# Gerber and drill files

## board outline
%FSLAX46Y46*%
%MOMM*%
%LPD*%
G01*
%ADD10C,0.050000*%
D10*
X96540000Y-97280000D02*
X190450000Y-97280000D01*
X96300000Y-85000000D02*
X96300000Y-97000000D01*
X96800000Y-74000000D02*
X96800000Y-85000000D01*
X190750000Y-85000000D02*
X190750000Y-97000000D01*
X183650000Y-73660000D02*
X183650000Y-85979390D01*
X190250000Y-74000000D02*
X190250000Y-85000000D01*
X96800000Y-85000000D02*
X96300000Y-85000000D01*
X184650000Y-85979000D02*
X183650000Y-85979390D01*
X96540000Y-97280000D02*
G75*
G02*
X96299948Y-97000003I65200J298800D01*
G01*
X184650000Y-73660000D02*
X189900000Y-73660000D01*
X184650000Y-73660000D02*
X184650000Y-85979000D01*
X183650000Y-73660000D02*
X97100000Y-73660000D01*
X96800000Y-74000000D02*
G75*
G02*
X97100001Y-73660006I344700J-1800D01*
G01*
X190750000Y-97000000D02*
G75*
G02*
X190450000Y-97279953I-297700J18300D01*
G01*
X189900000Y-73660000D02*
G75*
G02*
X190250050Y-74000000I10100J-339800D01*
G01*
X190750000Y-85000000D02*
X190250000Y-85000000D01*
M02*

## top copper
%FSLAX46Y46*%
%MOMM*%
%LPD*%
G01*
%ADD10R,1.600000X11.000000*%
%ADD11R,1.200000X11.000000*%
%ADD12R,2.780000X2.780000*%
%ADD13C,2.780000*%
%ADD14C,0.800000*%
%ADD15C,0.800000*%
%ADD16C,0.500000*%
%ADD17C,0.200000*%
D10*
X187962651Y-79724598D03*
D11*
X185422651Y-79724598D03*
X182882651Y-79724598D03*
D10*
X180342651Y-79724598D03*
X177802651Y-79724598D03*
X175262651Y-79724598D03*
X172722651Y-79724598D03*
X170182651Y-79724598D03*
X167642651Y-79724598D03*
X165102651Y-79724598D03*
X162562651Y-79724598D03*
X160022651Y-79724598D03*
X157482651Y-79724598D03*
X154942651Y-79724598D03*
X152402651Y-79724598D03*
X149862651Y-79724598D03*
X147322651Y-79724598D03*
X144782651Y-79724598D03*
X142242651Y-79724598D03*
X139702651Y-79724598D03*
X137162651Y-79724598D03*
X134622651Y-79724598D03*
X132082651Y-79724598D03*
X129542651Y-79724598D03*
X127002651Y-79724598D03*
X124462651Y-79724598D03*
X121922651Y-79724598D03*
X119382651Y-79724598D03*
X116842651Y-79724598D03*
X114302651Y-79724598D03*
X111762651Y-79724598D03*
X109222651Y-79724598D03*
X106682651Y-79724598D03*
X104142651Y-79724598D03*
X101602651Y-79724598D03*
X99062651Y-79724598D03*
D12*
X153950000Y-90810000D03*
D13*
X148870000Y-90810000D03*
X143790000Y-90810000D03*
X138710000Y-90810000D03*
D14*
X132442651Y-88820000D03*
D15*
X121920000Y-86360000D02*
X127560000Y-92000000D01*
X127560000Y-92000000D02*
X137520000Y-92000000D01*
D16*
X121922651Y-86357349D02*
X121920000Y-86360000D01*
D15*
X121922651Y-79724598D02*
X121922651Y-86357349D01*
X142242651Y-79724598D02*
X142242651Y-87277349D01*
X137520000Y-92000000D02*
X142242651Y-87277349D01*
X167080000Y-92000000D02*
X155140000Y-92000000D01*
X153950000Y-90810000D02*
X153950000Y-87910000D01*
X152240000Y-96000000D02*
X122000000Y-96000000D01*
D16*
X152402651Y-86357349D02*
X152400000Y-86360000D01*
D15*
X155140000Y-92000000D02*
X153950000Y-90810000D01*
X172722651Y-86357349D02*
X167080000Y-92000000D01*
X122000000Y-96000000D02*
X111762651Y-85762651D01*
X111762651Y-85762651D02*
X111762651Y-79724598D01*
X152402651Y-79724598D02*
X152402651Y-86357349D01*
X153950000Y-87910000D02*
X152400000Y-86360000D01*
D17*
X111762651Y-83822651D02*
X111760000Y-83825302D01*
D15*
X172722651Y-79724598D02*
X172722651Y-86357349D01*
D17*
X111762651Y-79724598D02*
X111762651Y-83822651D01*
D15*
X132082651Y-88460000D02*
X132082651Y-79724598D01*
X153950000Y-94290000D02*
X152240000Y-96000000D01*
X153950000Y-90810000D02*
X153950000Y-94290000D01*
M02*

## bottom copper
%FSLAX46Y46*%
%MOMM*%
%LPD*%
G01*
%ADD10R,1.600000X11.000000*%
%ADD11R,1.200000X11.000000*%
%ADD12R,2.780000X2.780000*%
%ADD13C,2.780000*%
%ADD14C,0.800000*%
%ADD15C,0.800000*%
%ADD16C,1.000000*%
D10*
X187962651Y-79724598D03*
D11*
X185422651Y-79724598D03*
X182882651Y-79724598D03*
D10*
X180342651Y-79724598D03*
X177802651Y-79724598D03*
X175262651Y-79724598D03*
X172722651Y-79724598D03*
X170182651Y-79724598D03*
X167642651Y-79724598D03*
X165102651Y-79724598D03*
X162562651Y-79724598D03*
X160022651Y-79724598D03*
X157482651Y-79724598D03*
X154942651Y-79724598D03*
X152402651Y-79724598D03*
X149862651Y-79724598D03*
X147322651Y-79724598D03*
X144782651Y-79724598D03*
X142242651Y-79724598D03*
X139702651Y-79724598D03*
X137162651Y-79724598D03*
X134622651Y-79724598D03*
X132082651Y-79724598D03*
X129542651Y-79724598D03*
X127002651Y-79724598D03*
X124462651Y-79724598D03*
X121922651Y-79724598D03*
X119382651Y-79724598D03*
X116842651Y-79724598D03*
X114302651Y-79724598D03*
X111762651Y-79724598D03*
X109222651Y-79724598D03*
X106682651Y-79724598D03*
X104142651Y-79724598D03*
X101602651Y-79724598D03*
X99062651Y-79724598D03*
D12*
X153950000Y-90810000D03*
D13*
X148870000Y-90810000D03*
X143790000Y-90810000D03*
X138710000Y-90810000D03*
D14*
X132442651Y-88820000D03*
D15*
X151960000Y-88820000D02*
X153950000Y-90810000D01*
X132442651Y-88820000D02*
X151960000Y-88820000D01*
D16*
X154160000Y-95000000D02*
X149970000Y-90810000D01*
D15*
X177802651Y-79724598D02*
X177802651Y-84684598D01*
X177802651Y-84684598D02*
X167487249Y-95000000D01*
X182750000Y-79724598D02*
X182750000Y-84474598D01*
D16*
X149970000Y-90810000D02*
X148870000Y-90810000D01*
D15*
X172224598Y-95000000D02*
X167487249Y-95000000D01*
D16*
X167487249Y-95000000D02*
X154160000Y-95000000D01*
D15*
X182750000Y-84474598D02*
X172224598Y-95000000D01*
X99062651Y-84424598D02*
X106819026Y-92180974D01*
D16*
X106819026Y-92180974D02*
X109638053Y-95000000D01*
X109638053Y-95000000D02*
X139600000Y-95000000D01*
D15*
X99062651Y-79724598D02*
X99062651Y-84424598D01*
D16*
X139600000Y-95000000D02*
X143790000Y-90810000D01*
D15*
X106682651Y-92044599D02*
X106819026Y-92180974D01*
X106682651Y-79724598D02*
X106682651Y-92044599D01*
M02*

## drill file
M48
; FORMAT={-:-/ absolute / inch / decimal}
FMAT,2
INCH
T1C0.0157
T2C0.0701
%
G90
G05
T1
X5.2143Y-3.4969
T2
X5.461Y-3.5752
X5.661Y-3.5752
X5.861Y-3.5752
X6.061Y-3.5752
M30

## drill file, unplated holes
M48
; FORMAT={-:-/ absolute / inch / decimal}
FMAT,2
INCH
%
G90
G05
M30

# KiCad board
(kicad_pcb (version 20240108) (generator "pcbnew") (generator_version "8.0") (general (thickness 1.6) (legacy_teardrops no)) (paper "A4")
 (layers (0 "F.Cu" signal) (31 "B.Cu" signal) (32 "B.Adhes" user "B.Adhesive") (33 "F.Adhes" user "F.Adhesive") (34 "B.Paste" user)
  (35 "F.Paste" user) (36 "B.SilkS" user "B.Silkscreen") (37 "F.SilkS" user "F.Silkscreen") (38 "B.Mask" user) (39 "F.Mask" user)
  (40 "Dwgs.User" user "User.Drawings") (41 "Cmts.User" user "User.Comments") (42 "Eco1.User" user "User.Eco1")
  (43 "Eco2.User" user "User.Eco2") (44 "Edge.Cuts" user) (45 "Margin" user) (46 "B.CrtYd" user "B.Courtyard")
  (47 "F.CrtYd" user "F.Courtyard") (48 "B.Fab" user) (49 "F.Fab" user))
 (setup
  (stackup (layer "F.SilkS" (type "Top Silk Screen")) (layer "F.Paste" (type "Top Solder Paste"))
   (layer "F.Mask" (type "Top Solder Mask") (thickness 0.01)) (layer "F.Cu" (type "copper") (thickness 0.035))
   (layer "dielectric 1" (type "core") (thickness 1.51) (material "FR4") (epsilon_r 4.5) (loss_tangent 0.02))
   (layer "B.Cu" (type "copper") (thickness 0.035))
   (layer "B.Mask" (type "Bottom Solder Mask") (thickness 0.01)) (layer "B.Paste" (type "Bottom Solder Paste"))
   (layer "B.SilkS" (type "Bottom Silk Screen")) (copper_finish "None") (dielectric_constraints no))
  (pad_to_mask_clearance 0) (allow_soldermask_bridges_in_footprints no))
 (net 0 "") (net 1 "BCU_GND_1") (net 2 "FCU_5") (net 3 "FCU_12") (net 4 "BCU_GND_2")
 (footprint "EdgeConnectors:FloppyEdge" (layer "F.Cu") (at 167.642651 87.344598)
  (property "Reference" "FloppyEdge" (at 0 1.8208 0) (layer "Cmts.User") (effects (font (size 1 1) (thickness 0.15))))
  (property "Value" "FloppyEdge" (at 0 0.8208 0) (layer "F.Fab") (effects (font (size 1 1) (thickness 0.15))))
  (pad "1" smd rect (at 20.32 -7.62) (size 1.6 11) (layers "F.Cu" "F.Paste" "F.Mask"))
  (pad "2" smd rect (at 20.32 -7.62) (size 1.6 11) (layers "B.Cu" "B.Paste" "B.Mask"))
  (pad "3" smd rect (at 17.78 -7.62) (size 1.2 11) (layers "F.Cu" "F.Paste" "F.Mask"))
  (pad "4" smd rect (at 17.78 -7.62) (size 1.2 11) (layers "B.Cu" "B.Paste" "B.Mask"))
  (pad "5" smd rect (at 15.24 -7.62) (size 1.2 11) (layers "F.Cu" "F.Paste" "F.Mask"))
  (pad "6" smd rect (at 15.24 -7.62) (size 1.2 11) (layers "B.Cu" "B.Paste" "B.Mask") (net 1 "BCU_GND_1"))
  (pad "7" smd rect (at 12.7 -7.62) (size 1.6 11) (layers "F.Cu" "F.Paste" "F.Mask"))
  (pad "8" smd rect (at 12.7 -7.62) (size 1.6 11) (layers "B.Cu" "B.Paste" "B.Mask"))
  (pad "9" smd rect (at 10.16 -7.62) (size 1.6 11) (layers "F.Cu" "F.Paste" "F.Mask"))
  (pad "10" smd rect (at 10.16 -7.62) (size 1.6 11) (layers "B.Cu" "B.Paste" "B.Mask") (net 1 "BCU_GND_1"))
  (pad "11" smd rect (at 7.62 -7.62) (size 1.6 11) (layers "F.Cu" "F.Paste" "F.Mask"))
  (pad "12" smd rect (at 7.62 -7.62) (size 1.6 11) (layers "B.Cu" "B.Paste" "B.Mask"))
  (pad "13" smd rect (at 5.08 -7.62) (size 1.6 11) (layers "F.Cu" "F.Paste" "F.Mask") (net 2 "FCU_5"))
  (pad "14" smd rect (at 5.08 -7.62) (size 1.6 11) (layers "B.Cu" "B.Paste" "B.Mask"))
  (pad "15" smd rect (at 2.54 -7.62) (size 1.6 11) (layers "F.Cu" "F.Paste" "F.Mask"))
  (pad "16" smd rect (at 2.54 -7.62) (size 1.6 11) (layers "B.Cu" "B.Paste" "B.Mask"))
  (pad "17" smd rect (at 0 -7.62) (size 1.6 11) (layers "F.Cu" "F.Paste" "F.Mask"))
  (pad "18" smd rect (at 0 -7.62) (size 1.6 11) (layers "B.Cu" "B.Paste" "B.Mask"))
  (pad "19" smd rect (at -2.54 -7.62) (size 1.6 11) (layers "F.Cu" "F.Paste" "F.Mask"))
  (pad "20" smd rect (at -2.54 -7.62) (size 1.6 11) (layers "B.Cu" "B.Paste" "B.Mask"))
  (pad "21" smd rect (at -5.08 -7.62) (size 1.6 11) (layers "F.Cu" "F.Paste" "F.Mask"))
  (pad "22" smd rect (at -5.08 -7.62) (size 1.6 11) (layers "B.Cu" "B.Paste" "B.Mask"))
  (pad "23" smd rect (at -7.62 -7.62) (size 1.6 11) (layers "F.Cu" "F.Paste" "F.Mask"))
  (pad "24" smd rect (at -7.62 -7.62) (size 1.6 11) (layers "B.Cu" "B.Paste" "B.Mask"))
  (pad "25" smd rect (at -10.16 -7.62) (size 1.6 11) (layers "F.Cu" "F.Paste" "F.Mask"))
  (pad "26" smd rect (at -10.16 -7.62) (size 1.6 11) (layers "B.Cu" "B.Paste" "B.Mask"))
  (pad "27" smd rect (at -12.7 -7.62) (size 1.6 11) (layers "F.Cu" "F.Paste" "F.Mask"))
  (pad "28" smd rect (at -12.7 -7.62) (size 1.6 11) (layers "B.Cu" "B.Paste" "B.Mask"))
  (pad "29" smd rect (at -15.24 -7.62) (size 1.6 11) (layers "F.Cu" "F.Paste" "F.Mask") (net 2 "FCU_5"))
  (pad "30" smd rect (at -15.24 -7.62) (size 1.6 11) (layers "B.Cu" "B.Paste" "B.Mask"))
  (pad "31" smd rect (at -17.78 -7.62) (size 1.6 11) (layers "F.Cu" "F.Paste" "F.Mask"))
  (pad "32" smd rect (at -17.78 -7.62) (size 1.6 11) (layers "B.Cu" "B.Paste" "B.Mask"))
  (pad "33" smd rect (at -20.32 -7.62) (size 1.6 11) (layers "F.Cu" "F.Paste" "F.Mask"))
  (pad "34" smd rect (at -20.32 -7.62) (size 1.6 11) (layers "B.Cu" "B.Paste" "B.Mask"))
  (pad "35" smd rect (at -22.86 -7.62) (size 1.6 11) (layers "F.Cu" "F.Paste" "F.Mask"))
  (pad "36" smd rect (at -22.86 -7.62) (size 1.6 11) (layers "B.Cu" "B.Paste" "B.Mask"))
  (pad "37" smd rect (at -25.4 -7.62) (size 1.6 11) (layers "F.Cu" "F.Paste" "F.Mask") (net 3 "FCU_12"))
  (pad "38" smd rect (at -25.4 -7.62) (size 1.6 11) (layers "B.Cu" "B.Paste" "B.Mask"))
  (pad "39" smd rect (at -27.94 -7.62) (size 1.6 11) (layers "F.Cu" "F.Paste" "F.Mask"))
  (pad "40" smd rect (at -27.94 -7.62) (size 1.6 11) (layers "B.Cu" "B.Paste" "B.Mask"))
  (pad "41" smd rect (at -30.48 -7.62) (size 1.6 11) (layers "F.Cu" "F.Paste" "F.Mask"))
  (pad "42" smd rect (at -30.48 -7.62) (size 1.6 11) (layers "B.Cu" "B.Paste" "B.Mask"))
  (pad "43" smd rect (at -33.02 -7.62) (size 1.6 11) (layers "F.Cu" "F.Paste" "F.Mask"))
  (pad "44" smd rect (at -33.02 -7.62) (size 1.6 11) (layers "B.Cu" "B.Paste" "B.Mask"))
  (pad "45" smd rect (at -35.56 -7.62) (size 1.6 11) (layers "F.Cu" "F.Paste" "F.Mask") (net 2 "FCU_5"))
  (pad "46" smd rect (at -35.56 -7.62) (size 1.6 11) (layers "B.Cu" "B.Paste" "B.Mask"))
  (pad "47" smd rect (at -38.1 -7.62) (size 1.6 11) (layers "F.Cu" "F.Paste" "F.Mask"))
  (pad "48" smd rect (at -38.1 -7.62) (size 1.6 11) (layers "B.Cu" "B.Paste" "B.Mask"))
  (pad "49" smd rect (at -40.64 -7.62) (size 1.6 11) (layers "F.Cu" "F.Paste" "F.Mask"))
  (pad "50" smd rect (at -40.64 -7.62) (size 1.6 11) (layers "B.Cu" "B.Paste" "B.Mask"))
  (pad "51" smd rect (at -43.18 -7.62) (size 1.6 11) (layers "F.Cu" "F.Paste" "F.Mask"))
  (pad "52" smd rect (at -43.18 -7.62) (size 1.6 11) (layers "B.Cu" "B.Paste" "B.Mask"))
  (pad "53" smd rect (at -45.72 -7.62) (size 1.6 11) (layers "F.Cu" "F.Paste" "F.Mask") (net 3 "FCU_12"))
  (pad "54" smd rect (at -45.72 -7.62) (size 1.6 11) (layers "B.Cu" "B.Paste" "B.Mask"))
  (pad "55" smd rect (at -48.26 -7.62) (size 1.6 11) (layers "F.Cu" "F.Paste" "F.Mask"))
  (pad "56" smd rect (at -48.26 -7.62) (size 1.6 11) (layers "B.Cu" "B.Paste" "B.Mask"))
  (pad "57" smd rect (at -50.8 -7.62) (size 1.6 11) (layers "F.Cu" "F.Paste" "F.Mask"))
  (pad "58" smd rect (at -50.8 -7.62) (size 1.6 11) (layers "B.Cu" "B.Paste" "B.Mask"))
  (pad "59" smd rect (at -53.34 -7.62) (size 1.6 11) (layers "F.Cu" "F.Paste" "F.Mask"))
  (pad "60" smd rect (at -53.34 -7.62) (size 1.6 11) (layers "B.Cu" "B.Paste" "B.Mask"))
  (pad "61" smd rect (at -55.88 -7.62) (size 1.6 11) (layers "F.Cu" "F.Paste" "F.Mask") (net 2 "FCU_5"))
  (pad "62" smd rect (at -55.88 -7.62) (size 1.6 11) (layers "B.Cu" "B.Paste" "B.Mask"))
  (pad "63" smd rect (at -58.42 -7.62) (size 1.6 11) (layers "F.Cu" "F.Paste" "F.Mask"))
  (pad "64" smd rect (at -58.42 -7.62) (size 1.6 11) (layers "B.Cu" "B.Paste" "B.Mask"))
  (pad "65" smd rect (at -60.96 -7.62) (size 1.6 11) (layers "F.Cu" "F.Paste" "F.Mask"))
  (pad "66" smd rect (at -60.96 -7.62) (size 1.6 11) (layers "B.Cu" "B.Paste" "B.Mask") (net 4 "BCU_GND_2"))
  (pad "67" smd rect (at -63.5 -7.62) (size 1.6 11) (layers "F.Cu" "F.Paste" "F.Mask"))
  (pad "68" smd rect (at -63.5 -7.62) (size 1.6 11) (layers "B.Cu" "B.Paste" "B.Mask"))
  (pad "69" smd rect (at -66.04 -7.62) (size 1.6 11) (layers "F.Cu" "F.Paste" "F.Mask"))
  (pad "70" smd rect (at -66.04 -7.62) (size 1.6 11) (layers "B.Cu" "B.Paste" "B.Mask"))
  (pad "71" smd rect (at -68.58 -7.62) (size 1.6 11) (layers "F.Cu" "F.Paste" "F.Mask"))
  (pad "72" smd rect (at -68.58 -7.62) (size 1.6 11) (layers "B.Cu" "B.Paste" "B.Mask") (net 4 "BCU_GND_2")))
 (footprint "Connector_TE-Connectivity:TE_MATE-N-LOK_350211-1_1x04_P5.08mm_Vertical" (layer "F.Cu") (at 153.95 90.81 180)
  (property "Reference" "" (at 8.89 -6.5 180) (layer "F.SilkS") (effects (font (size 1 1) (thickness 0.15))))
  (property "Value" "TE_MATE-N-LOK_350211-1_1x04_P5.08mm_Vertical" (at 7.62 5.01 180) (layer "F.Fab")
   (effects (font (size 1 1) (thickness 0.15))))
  (pad "1" thru_hole rect (at 0 0 180) (size 2.78 2.78) (drill 1.78) (layers "*.Cu" "*.Mask") (remove_unused_layers no) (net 2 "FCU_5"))
  (pad "2" thru_hole circle (at 5.08 0 180) (size 2.78 2.78) (drill 1.78) (layers "*.Cu" "*.Mask") (remove_unused_layers no)
   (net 1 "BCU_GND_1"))
  (pad "3" thru_hole circle (at 10.16 0 180) (size 2.78 2.78) (drill 1.78) (layers "*.Cu" "*.Mask") (remove_unused_layers no)
   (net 4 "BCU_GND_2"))
  (pad "4" thru_hole circle (at 15.24 0 180) (size 2.78 2.78) (drill 1.78) (layers "*.Cu" "*.Mask") (remove_unused_layers no)
   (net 3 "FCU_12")))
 (gr_line (start 96.54 97.28) (end 190.45 97.28) (stroke (width 0.05) (type solid)) (layer "Edge.Cuts"))
 (gr_line (start 96.3 85) (end 96.3 97) (stroke (width 0.05) (type solid)) (layer "Edge.Cuts"))
 (gr_line (start 96.8 74) (end 96.8 85) (stroke (width 0.05) (type solid)) (layer "Edge.Cuts"))
 (gr_line (start 190.75 85) (end 190.75 97) (stroke (width 0.05) (type solid)) (layer "Edge.Cuts"))
 (gr_line (start 183.65 73.66) (end 183.65 85.97939) (stroke (width 0.05) (type solid)) (layer "Edge.Cuts"))
 (gr_line (start 190.25 74) (end 190.25 85) (stroke (width 0.05) (type solid)) (layer "Edge.Cuts"))
 (gr_line (start 96.8 85) (end 96.3 85) (stroke (width 0.05) (type default)) (layer "Edge.Cuts"))
 (gr_line (start 184.65 85.979) (end 183.65 85.97939) (stroke (width 0.05) (type solid)) (layer "Edge.Cuts"))
 (gr_arc (start 96.54 97.28) (mid 96.373508 97.180791) (end 96.3 97) (stroke (width 0.05) (type default)) (layer "Edge.Cuts"))
 (gr_line (start 184.65 73.66) (end 189.9 73.66) (stroke (width 0.05) (type solid)) (layer "Edge.Cuts"))
 (gr_line (start 184.65 73.66) (end 184.65 85.979) (stroke (width 0.05) (type solid)) (layer "Edge.Cuts"))
 (gr_line (start 183.65 73.66) (end 97.1 73.66) (stroke (width 0.05) (type solid)) (layer "Edge.Cuts"))
 (gr_arc (start 96.8 74) (mid 96.885926 73.774065) (end 97.1 73.66) (stroke (width 0.05) (type default)) (layer "Edge.Cuts"))
 (gr_arc (start 190.75 97) (mid 190.657493 97.198198) (end 190.45 97.28) (stroke (width 0.05) (type default)) (layer "Edge.Cuts"))
 (gr_arc (start 189.9 73.66) (mid 190.146958 73.75597) (end 190.25 74) (stroke (width 0.05) (type default)) (layer "Edge.Cuts"))
 (gr_line (start 190.75 85) (end 190.25 85) (stroke (width 0.05) (type default)) (layer "Edge.Cuts"))
 (segment (start 121.92 86.36) (end 127.56 92) (width 0.8) (layer "F.Cu") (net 3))
 (segment (start 127.56 92) (end 137.52 92) (width 0.8) (layer "F.Cu") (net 3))
 (segment (start 121.922651 86.357349) (end 121.92 86.36) (width 0.5) (layer "F.Cu") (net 3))
 (segment (start 121.922651 79.724598) (end 121.922651 86.357349) (width 0.8) (layer "F.Cu") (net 3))
 (segment (start 142.242651 79.724598) (end 142.242651 87.277349) (width 0.8) (layer "F.Cu") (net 3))
 (segment (start 137.52 92) (end 142.242651 87.277349) (width 0.8) (layer "F.Cu") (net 3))
 (segment (start 167.08 92) (end 155.14 92) (width 0.8) (layer "F.Cu") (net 2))
 (segment (start 153.95 90.81) (end 153.95 87.91) (width 0.8) (layer "F.Cu") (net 2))
 (segment (start 152.24 96) (end 122 96) (width 0.8) (layer "F.Cu") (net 2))
 (segment (start 152.402651 86.357349) (end 152.4 86.36) (width 0.5) (layer "F.Cu") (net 2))
 (segment (start 155.14 92) (end 153.95 90.81) (width 0.8) (layer "F.Cu") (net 2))
 (segment (start 172.722651 86.357349) (end 167.08 92) (width 0.8) (layer "F.Cu") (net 2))
 (segment (start 122 96) (end 111.762651 85.762651) (width 0.8) (layer "F.Cu") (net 2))
 (segment (start 111.762651 85.762651) (end 111.762651 79.724598) (width 0.8) (layer "F.Cu") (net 2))
 (segment (start 152.402651 79.724598) (end 152.402651 86.357349) (width 0.8) (layer "F.Cu") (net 2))
 (segment (start 153.95 87.91) (end 152.4 86.36) (width 0.8) (layer "F.Cu") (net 2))
 (segment (start 111.762651 83.822651) (end 111.76 83.825302) (width 0.2) (layer "F.Cu") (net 2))
 (segment (start 172.722651 79.724598) (end 172.722651 86.357349) (width 0.8) (layer "F.Cu") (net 2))
 (segment (start 111.762651 79.724598) (end 111.762651 83.822651) (width 0.2) (layer "F.Cu") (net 2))
 (segment (start 132.082651 88.46) (end 132.082651 79.724598) (width 0.8) (layer "F.Cu") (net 2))
 (segment (start 153.95 94.29) (end 152.24 96) (width 0.8) (layer "F.Cu") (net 2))
 (segment (start 153.95 90.81) (end 153.95 94.29) (width 0.8) (layer "F.Cu") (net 2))
 (via blind (at 132.442651 88.82) (size 0.8) (drill 0.4) (layers "F.Cu" "B.Cu") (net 2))
 (segment (start 151.96 88.82) (end 153.95 90.81) (width 0.8) (layer "B.Cu") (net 2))
 (segment (start 132.442651 88.82) (end 151.96 88.82) (width 0.8) (layer "B.Cu") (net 2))
 (segment (start 154.16 95) (end 149.97 90.81) (width 1) (layer "B.Cu") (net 1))
 (segment (start 177.802651 79.724598) (end 177.802651 84.684598) (width 0.8) (layer "B.Cu") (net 1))
 (segment (start 177.802651 84.684598) (end 167.487249 95) (width 0.8) (layer "B.Cu") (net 1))
 (segment (start 182.75 79.724598) (end 182.75 84.474598) (width 0.8) (layer "B.Cu") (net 1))
 (segment (start 149.97 90.81) (end 148.87 90.81) (width 1) (layer "B.Cu") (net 1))
 (segment (start 172.224598 95) (end 167.487249 95) (width 0.8) (layer "B.Cu") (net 1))
 (segment (start 167.487249 95) (end 154.16 95) (width 1) (layer "B.Cu") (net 1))
 (segment (start 182.75 84.474598) (end 172.224598 95) (width 0.8) (layer "B.Cu") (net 1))
 (segment (start 99.062651 84.424598) (end 106.819026 92.180974) (width 0.8) (layer "B.Cu") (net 4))
 (segment (start 106.819026 92.180974) (end 109.638053 95) (width 1) (layer "B.Cu") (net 4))
 (segment (start 109.638053 95) (end 139.6 95) (width 1) (layer "B.Cu") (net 4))
 (segment (start 99.062651 79.724598) (end 99.062651 84.424598) (width 0.8) (layer "B.Cu") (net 4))
 (segment (start 139.6 95) (end 143.79 90.81) (width 1) (layer "B.Cu") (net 4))
 (segment (start 106.682651 92.044599) (end 106.819026 92.180974) (width 0.8) (layer "B.Cu") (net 4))
 (segment (start 106.682651 79.724598) (end 106.682651 92.044599) (width 0.8) (layer "B.Cu") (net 4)))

